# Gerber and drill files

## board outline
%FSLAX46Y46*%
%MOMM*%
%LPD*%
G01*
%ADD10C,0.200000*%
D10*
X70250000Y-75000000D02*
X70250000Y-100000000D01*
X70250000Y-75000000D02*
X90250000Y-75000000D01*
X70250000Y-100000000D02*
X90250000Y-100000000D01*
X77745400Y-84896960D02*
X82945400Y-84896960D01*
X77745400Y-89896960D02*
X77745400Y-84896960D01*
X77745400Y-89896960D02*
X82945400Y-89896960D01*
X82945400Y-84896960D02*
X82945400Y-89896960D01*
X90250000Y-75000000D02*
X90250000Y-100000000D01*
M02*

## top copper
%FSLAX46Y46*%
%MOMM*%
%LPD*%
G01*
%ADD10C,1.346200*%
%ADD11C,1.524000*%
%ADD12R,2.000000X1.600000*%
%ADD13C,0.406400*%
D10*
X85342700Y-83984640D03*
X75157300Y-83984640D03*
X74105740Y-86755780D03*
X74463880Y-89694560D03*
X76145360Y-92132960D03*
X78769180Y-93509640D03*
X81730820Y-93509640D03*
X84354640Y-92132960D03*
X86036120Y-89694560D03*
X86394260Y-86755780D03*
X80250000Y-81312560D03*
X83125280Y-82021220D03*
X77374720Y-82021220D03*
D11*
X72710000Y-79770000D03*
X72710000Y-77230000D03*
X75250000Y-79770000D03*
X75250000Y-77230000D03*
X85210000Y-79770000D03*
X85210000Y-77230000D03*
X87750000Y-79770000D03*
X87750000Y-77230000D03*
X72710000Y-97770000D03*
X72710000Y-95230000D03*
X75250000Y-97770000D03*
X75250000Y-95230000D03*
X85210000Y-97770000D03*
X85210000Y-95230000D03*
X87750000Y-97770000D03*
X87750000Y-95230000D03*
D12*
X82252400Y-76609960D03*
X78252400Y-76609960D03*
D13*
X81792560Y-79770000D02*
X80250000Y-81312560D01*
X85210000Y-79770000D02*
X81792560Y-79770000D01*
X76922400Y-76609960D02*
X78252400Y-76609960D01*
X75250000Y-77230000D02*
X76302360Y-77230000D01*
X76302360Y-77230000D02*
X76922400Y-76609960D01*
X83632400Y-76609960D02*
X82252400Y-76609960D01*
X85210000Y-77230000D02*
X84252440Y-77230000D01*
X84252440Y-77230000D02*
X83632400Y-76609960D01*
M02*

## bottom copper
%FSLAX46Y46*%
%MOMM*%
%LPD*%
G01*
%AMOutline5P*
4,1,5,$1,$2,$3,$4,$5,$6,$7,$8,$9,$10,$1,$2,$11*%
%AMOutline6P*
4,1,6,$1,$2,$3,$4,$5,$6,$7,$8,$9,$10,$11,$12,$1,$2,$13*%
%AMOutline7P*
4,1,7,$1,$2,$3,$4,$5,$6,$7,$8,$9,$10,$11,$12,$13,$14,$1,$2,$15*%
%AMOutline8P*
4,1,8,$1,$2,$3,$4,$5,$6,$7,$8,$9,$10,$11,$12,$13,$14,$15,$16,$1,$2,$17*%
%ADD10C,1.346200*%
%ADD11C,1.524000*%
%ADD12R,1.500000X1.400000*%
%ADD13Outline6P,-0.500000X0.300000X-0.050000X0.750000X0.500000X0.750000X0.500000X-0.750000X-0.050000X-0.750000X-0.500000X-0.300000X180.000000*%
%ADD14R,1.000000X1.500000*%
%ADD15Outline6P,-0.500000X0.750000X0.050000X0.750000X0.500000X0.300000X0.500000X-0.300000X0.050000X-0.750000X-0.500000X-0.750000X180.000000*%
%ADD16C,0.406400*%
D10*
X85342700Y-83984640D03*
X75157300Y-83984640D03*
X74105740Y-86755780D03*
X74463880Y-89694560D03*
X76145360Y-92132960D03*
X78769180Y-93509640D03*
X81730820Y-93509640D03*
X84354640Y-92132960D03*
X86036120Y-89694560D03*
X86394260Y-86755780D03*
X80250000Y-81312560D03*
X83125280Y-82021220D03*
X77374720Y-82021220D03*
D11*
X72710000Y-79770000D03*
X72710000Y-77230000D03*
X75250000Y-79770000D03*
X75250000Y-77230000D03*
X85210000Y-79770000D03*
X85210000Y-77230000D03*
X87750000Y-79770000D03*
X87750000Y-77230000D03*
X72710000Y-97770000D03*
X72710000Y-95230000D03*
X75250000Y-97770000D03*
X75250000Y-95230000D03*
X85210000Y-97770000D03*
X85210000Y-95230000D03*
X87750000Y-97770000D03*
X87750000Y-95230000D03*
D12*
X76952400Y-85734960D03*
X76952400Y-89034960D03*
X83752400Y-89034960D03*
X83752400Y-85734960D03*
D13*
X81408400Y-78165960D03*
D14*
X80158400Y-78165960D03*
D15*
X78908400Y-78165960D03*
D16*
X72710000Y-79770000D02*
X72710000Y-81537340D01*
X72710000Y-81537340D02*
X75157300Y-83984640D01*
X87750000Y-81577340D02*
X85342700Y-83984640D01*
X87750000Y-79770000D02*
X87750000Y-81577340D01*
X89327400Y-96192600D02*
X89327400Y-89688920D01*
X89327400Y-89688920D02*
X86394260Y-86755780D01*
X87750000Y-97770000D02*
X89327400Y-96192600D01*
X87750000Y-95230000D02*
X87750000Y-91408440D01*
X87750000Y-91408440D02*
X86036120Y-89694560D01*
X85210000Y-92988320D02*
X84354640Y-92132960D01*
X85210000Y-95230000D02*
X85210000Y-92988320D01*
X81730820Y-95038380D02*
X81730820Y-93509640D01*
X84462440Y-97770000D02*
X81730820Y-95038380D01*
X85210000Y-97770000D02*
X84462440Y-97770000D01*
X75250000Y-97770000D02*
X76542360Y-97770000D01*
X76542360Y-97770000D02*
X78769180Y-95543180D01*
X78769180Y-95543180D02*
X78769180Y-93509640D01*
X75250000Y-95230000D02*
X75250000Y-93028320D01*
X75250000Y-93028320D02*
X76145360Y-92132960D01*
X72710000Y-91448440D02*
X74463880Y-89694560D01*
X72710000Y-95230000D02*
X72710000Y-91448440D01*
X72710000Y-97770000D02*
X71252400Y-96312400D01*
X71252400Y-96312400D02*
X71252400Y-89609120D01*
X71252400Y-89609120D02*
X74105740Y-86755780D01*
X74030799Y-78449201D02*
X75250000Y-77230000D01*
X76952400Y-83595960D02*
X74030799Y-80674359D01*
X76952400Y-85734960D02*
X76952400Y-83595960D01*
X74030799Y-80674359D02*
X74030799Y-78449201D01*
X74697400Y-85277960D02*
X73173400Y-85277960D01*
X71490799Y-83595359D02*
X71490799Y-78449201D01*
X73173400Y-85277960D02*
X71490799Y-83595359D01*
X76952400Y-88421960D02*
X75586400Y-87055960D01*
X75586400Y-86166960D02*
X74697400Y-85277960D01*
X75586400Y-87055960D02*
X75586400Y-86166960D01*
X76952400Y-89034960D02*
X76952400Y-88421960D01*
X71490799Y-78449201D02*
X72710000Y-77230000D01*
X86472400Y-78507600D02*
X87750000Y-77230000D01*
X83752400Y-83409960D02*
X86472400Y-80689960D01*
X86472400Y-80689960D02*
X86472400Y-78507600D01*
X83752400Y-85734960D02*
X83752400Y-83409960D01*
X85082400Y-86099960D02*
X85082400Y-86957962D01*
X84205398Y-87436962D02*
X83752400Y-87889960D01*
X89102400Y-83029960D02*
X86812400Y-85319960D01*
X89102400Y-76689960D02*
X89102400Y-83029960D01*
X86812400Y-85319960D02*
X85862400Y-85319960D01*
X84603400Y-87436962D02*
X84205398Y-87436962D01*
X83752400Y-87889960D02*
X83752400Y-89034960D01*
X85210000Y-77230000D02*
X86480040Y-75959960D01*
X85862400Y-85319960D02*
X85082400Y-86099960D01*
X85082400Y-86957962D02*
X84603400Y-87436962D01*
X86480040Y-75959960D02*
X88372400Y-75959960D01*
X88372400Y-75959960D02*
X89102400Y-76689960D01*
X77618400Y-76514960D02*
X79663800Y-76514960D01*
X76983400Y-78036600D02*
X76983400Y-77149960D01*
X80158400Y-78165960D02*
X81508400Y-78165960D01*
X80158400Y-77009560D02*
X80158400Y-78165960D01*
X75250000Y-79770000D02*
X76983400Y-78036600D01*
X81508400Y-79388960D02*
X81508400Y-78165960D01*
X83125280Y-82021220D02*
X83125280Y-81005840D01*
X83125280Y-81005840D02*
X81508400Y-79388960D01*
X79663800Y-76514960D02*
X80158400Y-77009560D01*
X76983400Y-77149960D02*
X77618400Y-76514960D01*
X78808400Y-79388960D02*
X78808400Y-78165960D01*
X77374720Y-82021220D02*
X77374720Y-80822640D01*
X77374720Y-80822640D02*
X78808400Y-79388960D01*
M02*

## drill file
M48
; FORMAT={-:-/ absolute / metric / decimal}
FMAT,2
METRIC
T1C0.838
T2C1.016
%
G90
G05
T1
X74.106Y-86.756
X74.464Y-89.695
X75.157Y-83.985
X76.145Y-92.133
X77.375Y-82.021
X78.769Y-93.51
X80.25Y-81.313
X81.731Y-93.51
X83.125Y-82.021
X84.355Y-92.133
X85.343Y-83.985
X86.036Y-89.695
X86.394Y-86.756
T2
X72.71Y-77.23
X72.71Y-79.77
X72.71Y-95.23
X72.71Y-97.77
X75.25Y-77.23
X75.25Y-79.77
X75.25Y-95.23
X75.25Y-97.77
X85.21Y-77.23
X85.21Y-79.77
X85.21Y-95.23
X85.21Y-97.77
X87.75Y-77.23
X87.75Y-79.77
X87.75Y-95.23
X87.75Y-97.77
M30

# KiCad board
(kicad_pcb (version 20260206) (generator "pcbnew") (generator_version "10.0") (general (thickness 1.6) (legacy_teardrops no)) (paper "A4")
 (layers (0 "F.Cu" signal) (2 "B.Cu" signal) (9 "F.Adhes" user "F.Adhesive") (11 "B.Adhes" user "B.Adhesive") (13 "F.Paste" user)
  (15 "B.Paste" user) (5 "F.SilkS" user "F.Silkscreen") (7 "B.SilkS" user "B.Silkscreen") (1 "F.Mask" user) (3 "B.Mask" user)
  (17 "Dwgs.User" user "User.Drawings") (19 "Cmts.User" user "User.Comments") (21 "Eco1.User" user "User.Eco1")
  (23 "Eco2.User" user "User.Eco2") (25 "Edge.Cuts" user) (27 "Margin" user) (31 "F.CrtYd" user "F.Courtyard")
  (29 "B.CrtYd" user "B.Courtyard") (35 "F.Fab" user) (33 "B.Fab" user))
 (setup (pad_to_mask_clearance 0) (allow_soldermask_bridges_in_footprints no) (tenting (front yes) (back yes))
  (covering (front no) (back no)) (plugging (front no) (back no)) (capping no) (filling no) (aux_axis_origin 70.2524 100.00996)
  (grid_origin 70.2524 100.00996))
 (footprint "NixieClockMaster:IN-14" (layer "F.Cu") (at 80.25 87.5 180)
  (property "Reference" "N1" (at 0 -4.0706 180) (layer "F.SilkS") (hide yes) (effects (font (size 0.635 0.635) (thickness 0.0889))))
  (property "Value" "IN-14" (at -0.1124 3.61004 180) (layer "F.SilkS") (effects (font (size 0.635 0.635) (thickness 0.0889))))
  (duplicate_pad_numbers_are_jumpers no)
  (pad "0" thru_hole circle (at -5.0927 3.51536 180) (size 1.3462 1.3462) (drill 0.8382) (layers "*.Cu" "*.Mask") (remove_unused_layers no)
   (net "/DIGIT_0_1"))
  (pad "1" thru_hole circle (at 5.0927 3.51536 180) (size 1.3462 1.3462) (drill 0.8382) (layers "*.Cu" "*.Mask") (remove_unused_layers no)
   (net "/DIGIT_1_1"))
  (pad "2" thru_hole circle (at 6.14426 0.74422 180) (size 1.3462 1.3462) (drill 0.8382) (layers "*.Cu" "*.Mask") (remove_unused_layers no)
   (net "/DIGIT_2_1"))
  (pad "3" thru_hole circle (at 5.78612 -2.19456 180) (size 1.3462 1.3462) (drill 0.8382) (layers "*.Cu" "*.Mask") (remove_unused_layers no)
   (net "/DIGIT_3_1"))
  (pad "4" thru_hole circle (at 4.10464 -4.63296 180) (size 1.3462 1.3462) (drill 0.8382) (layers "*.Cu" "*.Mask") (remove_unused_layers no)
   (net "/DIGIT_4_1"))
  (pad "5" thru_hole circle (at 1.48082 -6.00964 180) (size 1.3462 1.3462) (drill 0.8382) (layers "*.Cu" "*.Mask") (remove_unused_layers no)
   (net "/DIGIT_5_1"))
  (pad "6" thru_hole circle (at -1.48082 -6.00964 180) (size 1.3462 1.3462) (drill 0.8382) (layers "*.Cu" "*.Mask")
   (remove_unused_layers no) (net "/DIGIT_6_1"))
  (pad "7" thru_hole circle (at -4.10464 -4.63296 180) (size 1.3462 1.3462) (drill 0.8382) (layers "*.Cu" "*.Mask")
   (remove_unused_layers no) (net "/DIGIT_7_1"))
  (pad "8" thru_hole circle (at -5.78612 -2.19456 180) (size 1.3462 1.3462) (drill 0.8382) (layers "*.Cu" "*.Mask")
   (remove_unused_layers no) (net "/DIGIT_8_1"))
  (pad "9" thru_hole circle (at -6.14426 0.74422 180) (size 1.3462 1.3462) (drill 0.8382) (layers "*.Cu" "*.Mask") (remove_unused_layers no)
   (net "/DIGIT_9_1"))
  (pad "A" thru_hole circle (at 0 6.18744 180) (size 1.3462 1.3462) (drill 0.8382) (layers "*.Cu" "*.Mask") (remove_unused_layers no)
   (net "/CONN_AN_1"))
  (pad "LHDP" thru_hole circle (at -2.87528 5.47878 180) (size 1.3462 1.3462) (drill 0.8382) (layers "*.Cu" "*.Mask")
   (remove_unused_layers no) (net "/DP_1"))
  (pad "RHDP" thru_hole circle (at 2.87528 5.47878 180) (size 1.3462 1.3462) (drill 0.8382) (layers "*.Cu" "*.Mask")
   (remove_unused_layers no) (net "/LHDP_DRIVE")))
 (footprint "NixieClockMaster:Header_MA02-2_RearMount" (layer "F.Cu") (at 75.25 78.5)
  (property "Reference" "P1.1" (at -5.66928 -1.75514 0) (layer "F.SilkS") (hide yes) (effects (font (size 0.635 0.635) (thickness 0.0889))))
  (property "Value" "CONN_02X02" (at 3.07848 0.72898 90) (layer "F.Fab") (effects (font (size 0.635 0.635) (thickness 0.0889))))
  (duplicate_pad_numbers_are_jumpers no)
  (pad "1" thru_hole circle (at -2.54 1.27) (size 1.524 1.524) (drill 1.016) (layers "*.Cu" "*.Mask") (remove_unused_layers no)
   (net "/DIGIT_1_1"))
  (pad "2" thru_hole circle (at -2.54 -1.27) (size 1.524 1.524) (drill 1.016) (layers "*.Cu" "*.Mask") (remove_unused_layers no)
   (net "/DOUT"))
  (pad "3" thru_hole circle (at 0 1.27) (size 1.524 1.524) (drill 1.016) (layers "*.Cu" "*.Mask") (remove_unused_layers no) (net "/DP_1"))
  (pad "4" thru_hole circle (at 0 -1.27) (size 1.524 1.524) (drill 1.016) (layers "*.Cu" "*.Mask") (remove_unused_layers no) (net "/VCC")))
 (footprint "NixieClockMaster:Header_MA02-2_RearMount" (layer "F.Cu") (at 87.75 78.5)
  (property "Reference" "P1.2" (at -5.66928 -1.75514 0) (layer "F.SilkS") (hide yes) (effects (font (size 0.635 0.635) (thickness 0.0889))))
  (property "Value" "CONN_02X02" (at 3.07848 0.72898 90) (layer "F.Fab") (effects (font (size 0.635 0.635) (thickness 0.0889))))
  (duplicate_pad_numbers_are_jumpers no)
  (pad "1" thru_hole circle (at -2.54 1.27) (size 1.524 1.524) (drill 1.016) (layers "*.Cu" "*.Mask") (remove_unused_layers no)
   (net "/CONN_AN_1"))
  (pad "2" thru_hole circle (at -2.54 -1.27) (size 1.524 1.524) (drill 1.016) (layers "*.Cu" "*.Mask") (remove_unused_layers no)
   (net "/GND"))
  (pad "3" thru_hole circle (at 0 1.27) (size 1.524 1.524) (drill 1.016) (layers "*.Cu" "*.Mask") (remove_unused_layers no)
   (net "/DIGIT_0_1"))
  (pad "4" thru_hole circle (at 0 -1.27) (size 1.524 1.524) (drill 1.016) (layers "*.Cu" "*.Mask") (remove_unused_layers no) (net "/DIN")))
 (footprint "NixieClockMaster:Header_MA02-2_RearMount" (layer "F.Cu") (at 75.25 96.5)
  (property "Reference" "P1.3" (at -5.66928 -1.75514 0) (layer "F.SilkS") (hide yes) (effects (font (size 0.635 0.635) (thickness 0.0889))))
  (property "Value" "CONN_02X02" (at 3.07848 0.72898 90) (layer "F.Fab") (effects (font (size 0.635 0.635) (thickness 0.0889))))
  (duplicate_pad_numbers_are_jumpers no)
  (pad "1" thru_hole circle (at -2.54 1.27) (size 1.524 1.524) (drill 1.016) (layers "*.Cu" "*.Mask") (remove_unused_layers no)
   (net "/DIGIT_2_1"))
  (pad "2" thru_hole circle (at -2.54 -1.27) (size 1.524 1.524) (drill 1.016) (layers "*.Cu" "*.Mask") (remove_unused_layers no)
   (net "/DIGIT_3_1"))
  (pad "3" thru_hole circle (at 0 1.27) (size 1.524 1.524) (drill 1.016) (layers "*.Cu" "*.Mask") (remove_unused_layers no)
   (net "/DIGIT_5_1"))
  (pad "4" thru_hole circle (at 0 -1.27) (size 1.524 1.524) (drill 1.016) (layers "*.Cu" "*.Mask") (remove_unused_layers no)
   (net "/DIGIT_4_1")))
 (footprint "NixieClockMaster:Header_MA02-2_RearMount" (layer "F.Cu") (at 87.75 96.5)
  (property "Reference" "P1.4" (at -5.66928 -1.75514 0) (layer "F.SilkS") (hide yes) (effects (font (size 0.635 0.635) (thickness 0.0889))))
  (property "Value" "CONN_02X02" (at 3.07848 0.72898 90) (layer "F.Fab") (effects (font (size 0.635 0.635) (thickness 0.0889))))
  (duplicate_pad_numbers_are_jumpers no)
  (pad "1" thru_hole circle (at -2.54 1.27) (size 1.524 1.524) (drill 1.016) (layers "*.Cu" "*.Mask") (remove_unused_layers no)
   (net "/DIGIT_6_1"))
  (pad "2" thru_hole circle (at -2.54 -1.27) (size 1.524 1.524) (drill 1.016) (layers "*.Cu" "*.Mask") (remove_unused_layers no)
   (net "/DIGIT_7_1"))
  (pad "3" thru_hole circle (at 0 1.27) (size 1.524 1.524) (drill 1.016) (layers "*.Cu" "*.Mask") (remove_unused_layers no)
   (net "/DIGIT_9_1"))
  (pad "4" thru_hole circle (at 0 -1.27) (size 1.524 1.524) (drill 1.016) (layers "*.Cu" "*.Mask") (remove_unused_layers no)
   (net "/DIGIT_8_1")))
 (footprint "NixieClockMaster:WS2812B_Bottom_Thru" (layer "F.Cu") (at 80.3524 87.38496 90)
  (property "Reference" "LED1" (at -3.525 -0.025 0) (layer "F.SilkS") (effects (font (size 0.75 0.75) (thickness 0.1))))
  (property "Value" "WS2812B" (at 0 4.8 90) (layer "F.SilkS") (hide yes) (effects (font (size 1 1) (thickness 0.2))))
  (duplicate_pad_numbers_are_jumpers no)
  (pad "1" smd rect (at 1.65 -3.4 90) (size 1.4 1.5) (layers "B.Cu" "B.Mask" "B.Paste") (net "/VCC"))
  (pad "2" smd rect (at -1.65 -3.4 90) (size 1.4 1.5) (layers "B.Cu" "B.Mask" "B.Paste") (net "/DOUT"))
  (pad "3" smd rect (at -1.65 3.4 90) (size 1.4 1.5) (layers "B.Cu" "B.Mask" "B.Paste") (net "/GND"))
  (pad "4" smd rect (at 1.65 3.4 90) (size 1.4 1.5) (layers "B.Cu" "B.Mask" "B.Paste") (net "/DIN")))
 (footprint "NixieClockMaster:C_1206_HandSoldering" (layer "F.Cu") (at 80.2524 76.60996 180)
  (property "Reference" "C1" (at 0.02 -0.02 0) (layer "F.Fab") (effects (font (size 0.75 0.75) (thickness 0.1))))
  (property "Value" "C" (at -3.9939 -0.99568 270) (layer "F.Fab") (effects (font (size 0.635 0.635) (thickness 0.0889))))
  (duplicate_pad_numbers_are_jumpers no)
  (pad "1" smd rect (at -2 0 180) (size 2 1.6) (layers "F.Cu" "F.Mask" "F.Paste") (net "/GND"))
  (pad "2" smd rect (at 2 0 180) (size 2 1.6) (layers "F.Cu" "F.Mask" "F.Paste") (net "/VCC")))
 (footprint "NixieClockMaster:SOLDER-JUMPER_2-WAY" (layer "B.Cu") (at 80.1584 78.16596 180)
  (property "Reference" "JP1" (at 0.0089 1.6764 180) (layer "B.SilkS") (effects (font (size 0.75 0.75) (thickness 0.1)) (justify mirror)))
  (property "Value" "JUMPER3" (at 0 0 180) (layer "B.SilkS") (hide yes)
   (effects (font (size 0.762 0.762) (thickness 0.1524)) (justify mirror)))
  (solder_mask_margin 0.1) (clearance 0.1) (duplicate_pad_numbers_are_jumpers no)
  (pad "1" smd roundrect (at -1.25 0 180) (size 1 1.5) (layers "B.Cu" "B.Mask") (roundrect_rratio 0) (chamfer_ratio 0.45)
   (chamfer top_left bottom_left) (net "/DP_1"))
  (pad "2" smd rect (at 0 0 180) (size 1 1.5) (layers "B.Cu" "B.Mask") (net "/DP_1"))
  (pad "3" smd roundrect (at 1.25 0 180) (size 1 1.5) (layers "B.Cu" "B.Mask") (roundrect_rratio 0) (chamfer_ratio 0.45)
   (chamfer top_right bottom_right) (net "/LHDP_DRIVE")))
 (gr_line (start 70.25 75) (end 70.25 100) (stroke (width 0.2) (type solid)) (layer "Edge.Cuts"))
 (gr_line (start 70.25 75) (end 90.25 75) (stroke (width 0.2) (type solid)) (layer "Edge.Cuts"))
 (gr_line (start 70.25 100) (end 90.25 100) (stroke (width 0.2) (type solid)) (layer "Edge.Cuts"))
 (gr_line (start 77.7454 84.89696) (end 82.9454 84.89696) (stroke (width 0.2) (type solid)) (layer "Edge.Cuts"))
 (gr_line (start 77.7454 89.89696) (end 77.7454 84.89696) (stroke (width 0.2) (type solid)) (layer "Edge.Cuts"))
 (gr_line (start 77.7454 89.89696) (end 82.9454 89.89696) (stroke (width 0.2) (type solid)) (layer "Edge.Cuts"))
 (gr_line (start 82.9454 84.89696) (end 82.9454 89.89696) (stroke (width 0.2) (type solid)) (layer "Edge.Cuts"))
 (gr_line (start 90.25 75) (end 90.25 100) (stroke (width 0.2) (type solid)) (layer "Edge.Cuts"))
 (segment (start 72.71 79.77) (end 72.71 81.53734) (width 0.4064) (layer "B.Cu") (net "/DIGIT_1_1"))
 (segment (start 72.71 81.53734) (end 75.1573 83.98464) (width 0.4064) (layer "B.Cu") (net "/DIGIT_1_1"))
 (segment (start 87.75 81.57734) (end 85.3427 83.98464) (width 0.4064) (layer "B.Cu") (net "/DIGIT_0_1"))
 (segment (start 87.75 79.77) (end 87.75 81.57734) (width 0.4064) (layer "B.Cu") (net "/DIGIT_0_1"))
 (segment (start 89.3274 96.1926) (end 89.3274 89.68892) (width 0.4064) (layer "B.Cu") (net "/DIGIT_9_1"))
 (segment (start 89.3274 89.68892) (end 86.39426 86.75578) (width 0.4064) (layer "B.Cu") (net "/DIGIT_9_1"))
 (segment (start 87.75 97.77) (end 89.3274 96.1926) (width 0.4064) (layer "B.Cu") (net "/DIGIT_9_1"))
 (segment (start 87.75 95.23) (end 87.75 91.40844) (width 0.4064) (layer "B.Cu") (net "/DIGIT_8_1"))
 (segment (start 87.75 91.40844) (end 86.03612 89.69456) (width 0.4064) (layer "B.Cu") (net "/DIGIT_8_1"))
 (segment (start 85.21 92.98832) (end 84.35464 92.13296) (width 0.4064) (layer "B.Cu") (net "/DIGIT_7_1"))
 (segment (start 85.21 95.23) (end 85.21 92.98832) (width 0.4064) (layer "B.Cu") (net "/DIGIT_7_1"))
 (segment (start 81.73082 95.03838) (end 81.73082 93.50964) (width 0.4064) (layer "B.Cu") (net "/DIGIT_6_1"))
 (segment (start 84.46244 97.77) (end 81.73082 95.03838) (width 0.4064) (layer "B.Cu") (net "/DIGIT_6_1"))
 (segment (start 85.21 97.77) (end 84.46244 97.77) (width 0.4064) (layer "B.Cu") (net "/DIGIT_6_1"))
 (segment (start 75.25 97.77) (end 76.54236 97.77) (width 0.4064) (layer "B.Cu") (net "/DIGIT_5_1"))
 (segment (start 76.54236 97.77) (end 78.76918 95.54318) (width 0.4064) (layer "B.Cu") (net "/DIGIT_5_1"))
 (segment (start 78.76918 95.54318) (end 78.76918 93.50964) (width 0.4064) (layer "B.Cu") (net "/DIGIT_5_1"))
 (segment (start 75.25 95.23) (end 75.25 93.02832) (width 0.4064) (layer "B.Cu") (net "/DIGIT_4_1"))
 (segment (start 75.25 93.02832) (end 76.14536 92.13296) (width 0.4064) (layer "B.Cu") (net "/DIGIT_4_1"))
 (segment (start 72.71 91.44844) (end 74.46388 89.69456) (width 0.4064) (layer "B.Cu") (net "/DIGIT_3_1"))
 (segment (start 72.71 95.23) (end 72.71 91.44844) (width 0.4064) (layer "B.Cu") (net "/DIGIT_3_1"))
 (segment (start 72.71 97.77) (end 71.2524 96.3124) (width 0.4064) (layer "B.Cu") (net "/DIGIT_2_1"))
 (segment (start 71.2524 96.3124) (end 71.2524 89.60912) (width 0.4064) (layer "B.Cu") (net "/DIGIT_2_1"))
 (segment (start 71.2524 89.60912) (end 74.10574 86.75578) (width 0.4064) (layer "B.Cu") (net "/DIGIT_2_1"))
 (segment (start 81.79256 79.77) (end 80.25 81.31256) (width 0.4064) (layer "F.Cu") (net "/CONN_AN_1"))
 (segment (start 85.21 79.77) (end 81.79256 79.77) (width 0.4064) (layer "F.Cu") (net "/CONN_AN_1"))
 (segment (start 76.9224 76.60996) (end 78.2524 76.60996) (width 0.4064) (layer "F.Cu") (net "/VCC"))
 (segment (start 75.25 77.23) (end 76.30236 77.23) (width 0.4064) (layer "F.Cu") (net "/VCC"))
 (segment (start 76.30236 77.23) (end 76.9224 76.60996) (width 0.4064) (layer "F.Cu") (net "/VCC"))
 (segment (start 74.030799 78.449201) (end 75.25 77.23) (width 0.4064) (layer "B.Cu") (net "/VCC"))
 (segment (start 76.9524 83.59596) (end 74.030799 80.674359) (width 0.4064) (layer "B.Cu") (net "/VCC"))
 (segment (start 76.9524 85.73496) (end 76.9524 83.59596) (width 0.4064) (layer "B.Cu") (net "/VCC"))
 (segment (start 74.030799 80.674359) (end 74.030799 78.449201) (width 0.4064) (layer "B.Cu") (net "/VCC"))
 (segment (start 74.6974 85.27796) (end 73.1734 85.27796) (width 0.4064) (layer "B.Cu") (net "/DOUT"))
 (segment (start 71.490799 83.595359) (end 71.490799 78.449201) (width 0.4064) (layer "B.Cu") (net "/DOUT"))
 (segment (start 73.1734 85.27796) (end 71.490799 83.595359) (width 0.4064) (layer "B.Cu") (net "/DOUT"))
 (segment (start 76.9524 88.42196) (end 75.5864 87.05596) (width 0.4064) (layer "B.Cu") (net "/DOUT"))
 (segment (start 75.5864 86.16696) (end 74.6974 85.27796) (width 0.4064) (layer "B.Cu") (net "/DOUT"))
 (segment (start 75.5864 87.05596) (end 75.5864 86.16696) (width 0.4064) (layer "B.Cu") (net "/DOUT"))
 (segment (start 76.9524 89.03496) (end 76.9524 88.42196) (width 0.4064) (layer "B.Cu") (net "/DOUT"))
 (segment (start 71.490799 78.449201) (end 72.71 77.23) (width 0.4064) (layer "B.Cu") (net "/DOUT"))
 (segment (start 86.4724 78.5076) (end 87.75 77.23) (width 0.4064) (layer "B.Cu") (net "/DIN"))
 (segment (start 83.7524 83.40996) (end 86.4724 80.68996) (width 0.4064) (layer "B.Cu") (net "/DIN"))
 (segment (start 86.4724 80.68996) (end 86.4724 78.5076) (width 0.4064) (layer "B.Cu") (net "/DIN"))
 (segment (start 83.7524 85.73496) (end 83.7524 83.40996) (width 0.4064) (layer "B.Cu") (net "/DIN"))
 (segment (start 83.6324 76.60996) (end 82.2524 76.60996) (width 0.4064) (layer "F.Cu") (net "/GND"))
 (segment (start 85.21 77.23) (end 84.25244 77.23) (width 0.4064) (layer "F.Cu") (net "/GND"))
 (segment (start 84.25244 77.23) (end 83.6324 76.60996) (width 0.4064) (layer "F.Cu") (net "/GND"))
 (segment (start 85.0824 86.09996) (end 85.0824 86.957962) (width 0.4064) (layer "B.Cu") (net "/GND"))
 (segment (start 84.205398 87.436962) (end 83.7524 87.88996) (width 0.4064) (layer "B.Cu") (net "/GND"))
 (segment (start 89.1024 83.02996) (end 86.8124 85.31996) (width 0.4064) (layer "B.Cu") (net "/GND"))
 (segment (start 89.1024 76.68996) (end 89.1024 83.02996) (width 0.4064) (layer "B.Cu") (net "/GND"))
 (segment (start 86.8124 85.31996) (end 85.8624 85.31996) (width 0.4064) (layer "B.Cu") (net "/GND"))
 (segment (start 84.6034 87.436962) (end 84.205398 87.436962) (width 0.4064) (layer "B.Cu") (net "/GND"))
 (segment (start 83.7524 87.88996) (end 83.7524 89.03496) (width 0.4064) (layer "B.Cu") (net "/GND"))
 (segment (start 85.21 77.23) (end 86.48004 75.95996) (width 0.4064) (layer "B.Cu") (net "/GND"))
 (segment (start 85.8624 85.31996) (end 85.0824 86.09996) (width 0.4064) (layer "B.Cu") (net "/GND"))
 (segment (start 85.0824 86.957962) (end 84.6034 87.436962) (width 0.4064) (layer "B.Cu") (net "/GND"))
 (segment (start 86.48004 75.95996) (end 88.3724 75.95996) (width 0.4064) (layer "B.Cu") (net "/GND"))
 (segment (start 88.3724 75.95996) (end 89.1024 76.68996) (width 0.4064) (layer "B.Cu") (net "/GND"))
 (segment (start 77.6184 76.51496) (end 79.6638 76.51496) (width 0.4064) (layer "B.Cu") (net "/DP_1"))
 (segment (start 76.9834 78.0366) (end 76.9834 77.14996) (width 0.4064) (layer "B.Cu") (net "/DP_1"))
 (segment (start 80.1584 78.16596) (end 81.5084 78.16596) (width 0.4064) (layer "B.Cu") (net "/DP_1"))
 (segment (start 80.1584 77.00956) (end 80.1584 78.16596) (width 0.4064) (layer "B.Cu") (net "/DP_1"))
 (segment (start 75.25 79.77) (end 76.9834 78.0366) (width 0.4064) (layer "B.Cu") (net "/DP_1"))
 (segment (start 81.5084 79.38896) (end 81.5084 78.16596) (width 0.4064) (layer "B.Cu") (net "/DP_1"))
 (segment (start 83.12528 82.02122) (end 83.12528 81.00584) (width 0.4064) (layer "B.Cu") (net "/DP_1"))
 (segment (start 83.12528 81.00584) (end 81.5084 79.38896) (width 0.4064) (layer "B.Cu") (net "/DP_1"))
 (segment (start 79.6638 76.51496) (end 80.1584 77.00956) (width 0.4064) (layer "B.Cu") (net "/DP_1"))
 (segment (start 76.9834 77.14996) (end 77.6184 76.51496) (width 0.4064) (layer "B.Cu") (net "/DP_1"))
 (segment (start 78.8084 79.38896) (end 78.8084 78.16596) (width 0.4064) (layer "B.Cu") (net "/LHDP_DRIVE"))
 (segment (start 77.37472 82.02122) (end 77.37472 80.82264) (width 0.4064) (layer "B.Cu") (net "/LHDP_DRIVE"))
 (segment (start 77.37472 80.82264) (end 78.8084 79.38896) (width 0.4064) (layer "B.Cu") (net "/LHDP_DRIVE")))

